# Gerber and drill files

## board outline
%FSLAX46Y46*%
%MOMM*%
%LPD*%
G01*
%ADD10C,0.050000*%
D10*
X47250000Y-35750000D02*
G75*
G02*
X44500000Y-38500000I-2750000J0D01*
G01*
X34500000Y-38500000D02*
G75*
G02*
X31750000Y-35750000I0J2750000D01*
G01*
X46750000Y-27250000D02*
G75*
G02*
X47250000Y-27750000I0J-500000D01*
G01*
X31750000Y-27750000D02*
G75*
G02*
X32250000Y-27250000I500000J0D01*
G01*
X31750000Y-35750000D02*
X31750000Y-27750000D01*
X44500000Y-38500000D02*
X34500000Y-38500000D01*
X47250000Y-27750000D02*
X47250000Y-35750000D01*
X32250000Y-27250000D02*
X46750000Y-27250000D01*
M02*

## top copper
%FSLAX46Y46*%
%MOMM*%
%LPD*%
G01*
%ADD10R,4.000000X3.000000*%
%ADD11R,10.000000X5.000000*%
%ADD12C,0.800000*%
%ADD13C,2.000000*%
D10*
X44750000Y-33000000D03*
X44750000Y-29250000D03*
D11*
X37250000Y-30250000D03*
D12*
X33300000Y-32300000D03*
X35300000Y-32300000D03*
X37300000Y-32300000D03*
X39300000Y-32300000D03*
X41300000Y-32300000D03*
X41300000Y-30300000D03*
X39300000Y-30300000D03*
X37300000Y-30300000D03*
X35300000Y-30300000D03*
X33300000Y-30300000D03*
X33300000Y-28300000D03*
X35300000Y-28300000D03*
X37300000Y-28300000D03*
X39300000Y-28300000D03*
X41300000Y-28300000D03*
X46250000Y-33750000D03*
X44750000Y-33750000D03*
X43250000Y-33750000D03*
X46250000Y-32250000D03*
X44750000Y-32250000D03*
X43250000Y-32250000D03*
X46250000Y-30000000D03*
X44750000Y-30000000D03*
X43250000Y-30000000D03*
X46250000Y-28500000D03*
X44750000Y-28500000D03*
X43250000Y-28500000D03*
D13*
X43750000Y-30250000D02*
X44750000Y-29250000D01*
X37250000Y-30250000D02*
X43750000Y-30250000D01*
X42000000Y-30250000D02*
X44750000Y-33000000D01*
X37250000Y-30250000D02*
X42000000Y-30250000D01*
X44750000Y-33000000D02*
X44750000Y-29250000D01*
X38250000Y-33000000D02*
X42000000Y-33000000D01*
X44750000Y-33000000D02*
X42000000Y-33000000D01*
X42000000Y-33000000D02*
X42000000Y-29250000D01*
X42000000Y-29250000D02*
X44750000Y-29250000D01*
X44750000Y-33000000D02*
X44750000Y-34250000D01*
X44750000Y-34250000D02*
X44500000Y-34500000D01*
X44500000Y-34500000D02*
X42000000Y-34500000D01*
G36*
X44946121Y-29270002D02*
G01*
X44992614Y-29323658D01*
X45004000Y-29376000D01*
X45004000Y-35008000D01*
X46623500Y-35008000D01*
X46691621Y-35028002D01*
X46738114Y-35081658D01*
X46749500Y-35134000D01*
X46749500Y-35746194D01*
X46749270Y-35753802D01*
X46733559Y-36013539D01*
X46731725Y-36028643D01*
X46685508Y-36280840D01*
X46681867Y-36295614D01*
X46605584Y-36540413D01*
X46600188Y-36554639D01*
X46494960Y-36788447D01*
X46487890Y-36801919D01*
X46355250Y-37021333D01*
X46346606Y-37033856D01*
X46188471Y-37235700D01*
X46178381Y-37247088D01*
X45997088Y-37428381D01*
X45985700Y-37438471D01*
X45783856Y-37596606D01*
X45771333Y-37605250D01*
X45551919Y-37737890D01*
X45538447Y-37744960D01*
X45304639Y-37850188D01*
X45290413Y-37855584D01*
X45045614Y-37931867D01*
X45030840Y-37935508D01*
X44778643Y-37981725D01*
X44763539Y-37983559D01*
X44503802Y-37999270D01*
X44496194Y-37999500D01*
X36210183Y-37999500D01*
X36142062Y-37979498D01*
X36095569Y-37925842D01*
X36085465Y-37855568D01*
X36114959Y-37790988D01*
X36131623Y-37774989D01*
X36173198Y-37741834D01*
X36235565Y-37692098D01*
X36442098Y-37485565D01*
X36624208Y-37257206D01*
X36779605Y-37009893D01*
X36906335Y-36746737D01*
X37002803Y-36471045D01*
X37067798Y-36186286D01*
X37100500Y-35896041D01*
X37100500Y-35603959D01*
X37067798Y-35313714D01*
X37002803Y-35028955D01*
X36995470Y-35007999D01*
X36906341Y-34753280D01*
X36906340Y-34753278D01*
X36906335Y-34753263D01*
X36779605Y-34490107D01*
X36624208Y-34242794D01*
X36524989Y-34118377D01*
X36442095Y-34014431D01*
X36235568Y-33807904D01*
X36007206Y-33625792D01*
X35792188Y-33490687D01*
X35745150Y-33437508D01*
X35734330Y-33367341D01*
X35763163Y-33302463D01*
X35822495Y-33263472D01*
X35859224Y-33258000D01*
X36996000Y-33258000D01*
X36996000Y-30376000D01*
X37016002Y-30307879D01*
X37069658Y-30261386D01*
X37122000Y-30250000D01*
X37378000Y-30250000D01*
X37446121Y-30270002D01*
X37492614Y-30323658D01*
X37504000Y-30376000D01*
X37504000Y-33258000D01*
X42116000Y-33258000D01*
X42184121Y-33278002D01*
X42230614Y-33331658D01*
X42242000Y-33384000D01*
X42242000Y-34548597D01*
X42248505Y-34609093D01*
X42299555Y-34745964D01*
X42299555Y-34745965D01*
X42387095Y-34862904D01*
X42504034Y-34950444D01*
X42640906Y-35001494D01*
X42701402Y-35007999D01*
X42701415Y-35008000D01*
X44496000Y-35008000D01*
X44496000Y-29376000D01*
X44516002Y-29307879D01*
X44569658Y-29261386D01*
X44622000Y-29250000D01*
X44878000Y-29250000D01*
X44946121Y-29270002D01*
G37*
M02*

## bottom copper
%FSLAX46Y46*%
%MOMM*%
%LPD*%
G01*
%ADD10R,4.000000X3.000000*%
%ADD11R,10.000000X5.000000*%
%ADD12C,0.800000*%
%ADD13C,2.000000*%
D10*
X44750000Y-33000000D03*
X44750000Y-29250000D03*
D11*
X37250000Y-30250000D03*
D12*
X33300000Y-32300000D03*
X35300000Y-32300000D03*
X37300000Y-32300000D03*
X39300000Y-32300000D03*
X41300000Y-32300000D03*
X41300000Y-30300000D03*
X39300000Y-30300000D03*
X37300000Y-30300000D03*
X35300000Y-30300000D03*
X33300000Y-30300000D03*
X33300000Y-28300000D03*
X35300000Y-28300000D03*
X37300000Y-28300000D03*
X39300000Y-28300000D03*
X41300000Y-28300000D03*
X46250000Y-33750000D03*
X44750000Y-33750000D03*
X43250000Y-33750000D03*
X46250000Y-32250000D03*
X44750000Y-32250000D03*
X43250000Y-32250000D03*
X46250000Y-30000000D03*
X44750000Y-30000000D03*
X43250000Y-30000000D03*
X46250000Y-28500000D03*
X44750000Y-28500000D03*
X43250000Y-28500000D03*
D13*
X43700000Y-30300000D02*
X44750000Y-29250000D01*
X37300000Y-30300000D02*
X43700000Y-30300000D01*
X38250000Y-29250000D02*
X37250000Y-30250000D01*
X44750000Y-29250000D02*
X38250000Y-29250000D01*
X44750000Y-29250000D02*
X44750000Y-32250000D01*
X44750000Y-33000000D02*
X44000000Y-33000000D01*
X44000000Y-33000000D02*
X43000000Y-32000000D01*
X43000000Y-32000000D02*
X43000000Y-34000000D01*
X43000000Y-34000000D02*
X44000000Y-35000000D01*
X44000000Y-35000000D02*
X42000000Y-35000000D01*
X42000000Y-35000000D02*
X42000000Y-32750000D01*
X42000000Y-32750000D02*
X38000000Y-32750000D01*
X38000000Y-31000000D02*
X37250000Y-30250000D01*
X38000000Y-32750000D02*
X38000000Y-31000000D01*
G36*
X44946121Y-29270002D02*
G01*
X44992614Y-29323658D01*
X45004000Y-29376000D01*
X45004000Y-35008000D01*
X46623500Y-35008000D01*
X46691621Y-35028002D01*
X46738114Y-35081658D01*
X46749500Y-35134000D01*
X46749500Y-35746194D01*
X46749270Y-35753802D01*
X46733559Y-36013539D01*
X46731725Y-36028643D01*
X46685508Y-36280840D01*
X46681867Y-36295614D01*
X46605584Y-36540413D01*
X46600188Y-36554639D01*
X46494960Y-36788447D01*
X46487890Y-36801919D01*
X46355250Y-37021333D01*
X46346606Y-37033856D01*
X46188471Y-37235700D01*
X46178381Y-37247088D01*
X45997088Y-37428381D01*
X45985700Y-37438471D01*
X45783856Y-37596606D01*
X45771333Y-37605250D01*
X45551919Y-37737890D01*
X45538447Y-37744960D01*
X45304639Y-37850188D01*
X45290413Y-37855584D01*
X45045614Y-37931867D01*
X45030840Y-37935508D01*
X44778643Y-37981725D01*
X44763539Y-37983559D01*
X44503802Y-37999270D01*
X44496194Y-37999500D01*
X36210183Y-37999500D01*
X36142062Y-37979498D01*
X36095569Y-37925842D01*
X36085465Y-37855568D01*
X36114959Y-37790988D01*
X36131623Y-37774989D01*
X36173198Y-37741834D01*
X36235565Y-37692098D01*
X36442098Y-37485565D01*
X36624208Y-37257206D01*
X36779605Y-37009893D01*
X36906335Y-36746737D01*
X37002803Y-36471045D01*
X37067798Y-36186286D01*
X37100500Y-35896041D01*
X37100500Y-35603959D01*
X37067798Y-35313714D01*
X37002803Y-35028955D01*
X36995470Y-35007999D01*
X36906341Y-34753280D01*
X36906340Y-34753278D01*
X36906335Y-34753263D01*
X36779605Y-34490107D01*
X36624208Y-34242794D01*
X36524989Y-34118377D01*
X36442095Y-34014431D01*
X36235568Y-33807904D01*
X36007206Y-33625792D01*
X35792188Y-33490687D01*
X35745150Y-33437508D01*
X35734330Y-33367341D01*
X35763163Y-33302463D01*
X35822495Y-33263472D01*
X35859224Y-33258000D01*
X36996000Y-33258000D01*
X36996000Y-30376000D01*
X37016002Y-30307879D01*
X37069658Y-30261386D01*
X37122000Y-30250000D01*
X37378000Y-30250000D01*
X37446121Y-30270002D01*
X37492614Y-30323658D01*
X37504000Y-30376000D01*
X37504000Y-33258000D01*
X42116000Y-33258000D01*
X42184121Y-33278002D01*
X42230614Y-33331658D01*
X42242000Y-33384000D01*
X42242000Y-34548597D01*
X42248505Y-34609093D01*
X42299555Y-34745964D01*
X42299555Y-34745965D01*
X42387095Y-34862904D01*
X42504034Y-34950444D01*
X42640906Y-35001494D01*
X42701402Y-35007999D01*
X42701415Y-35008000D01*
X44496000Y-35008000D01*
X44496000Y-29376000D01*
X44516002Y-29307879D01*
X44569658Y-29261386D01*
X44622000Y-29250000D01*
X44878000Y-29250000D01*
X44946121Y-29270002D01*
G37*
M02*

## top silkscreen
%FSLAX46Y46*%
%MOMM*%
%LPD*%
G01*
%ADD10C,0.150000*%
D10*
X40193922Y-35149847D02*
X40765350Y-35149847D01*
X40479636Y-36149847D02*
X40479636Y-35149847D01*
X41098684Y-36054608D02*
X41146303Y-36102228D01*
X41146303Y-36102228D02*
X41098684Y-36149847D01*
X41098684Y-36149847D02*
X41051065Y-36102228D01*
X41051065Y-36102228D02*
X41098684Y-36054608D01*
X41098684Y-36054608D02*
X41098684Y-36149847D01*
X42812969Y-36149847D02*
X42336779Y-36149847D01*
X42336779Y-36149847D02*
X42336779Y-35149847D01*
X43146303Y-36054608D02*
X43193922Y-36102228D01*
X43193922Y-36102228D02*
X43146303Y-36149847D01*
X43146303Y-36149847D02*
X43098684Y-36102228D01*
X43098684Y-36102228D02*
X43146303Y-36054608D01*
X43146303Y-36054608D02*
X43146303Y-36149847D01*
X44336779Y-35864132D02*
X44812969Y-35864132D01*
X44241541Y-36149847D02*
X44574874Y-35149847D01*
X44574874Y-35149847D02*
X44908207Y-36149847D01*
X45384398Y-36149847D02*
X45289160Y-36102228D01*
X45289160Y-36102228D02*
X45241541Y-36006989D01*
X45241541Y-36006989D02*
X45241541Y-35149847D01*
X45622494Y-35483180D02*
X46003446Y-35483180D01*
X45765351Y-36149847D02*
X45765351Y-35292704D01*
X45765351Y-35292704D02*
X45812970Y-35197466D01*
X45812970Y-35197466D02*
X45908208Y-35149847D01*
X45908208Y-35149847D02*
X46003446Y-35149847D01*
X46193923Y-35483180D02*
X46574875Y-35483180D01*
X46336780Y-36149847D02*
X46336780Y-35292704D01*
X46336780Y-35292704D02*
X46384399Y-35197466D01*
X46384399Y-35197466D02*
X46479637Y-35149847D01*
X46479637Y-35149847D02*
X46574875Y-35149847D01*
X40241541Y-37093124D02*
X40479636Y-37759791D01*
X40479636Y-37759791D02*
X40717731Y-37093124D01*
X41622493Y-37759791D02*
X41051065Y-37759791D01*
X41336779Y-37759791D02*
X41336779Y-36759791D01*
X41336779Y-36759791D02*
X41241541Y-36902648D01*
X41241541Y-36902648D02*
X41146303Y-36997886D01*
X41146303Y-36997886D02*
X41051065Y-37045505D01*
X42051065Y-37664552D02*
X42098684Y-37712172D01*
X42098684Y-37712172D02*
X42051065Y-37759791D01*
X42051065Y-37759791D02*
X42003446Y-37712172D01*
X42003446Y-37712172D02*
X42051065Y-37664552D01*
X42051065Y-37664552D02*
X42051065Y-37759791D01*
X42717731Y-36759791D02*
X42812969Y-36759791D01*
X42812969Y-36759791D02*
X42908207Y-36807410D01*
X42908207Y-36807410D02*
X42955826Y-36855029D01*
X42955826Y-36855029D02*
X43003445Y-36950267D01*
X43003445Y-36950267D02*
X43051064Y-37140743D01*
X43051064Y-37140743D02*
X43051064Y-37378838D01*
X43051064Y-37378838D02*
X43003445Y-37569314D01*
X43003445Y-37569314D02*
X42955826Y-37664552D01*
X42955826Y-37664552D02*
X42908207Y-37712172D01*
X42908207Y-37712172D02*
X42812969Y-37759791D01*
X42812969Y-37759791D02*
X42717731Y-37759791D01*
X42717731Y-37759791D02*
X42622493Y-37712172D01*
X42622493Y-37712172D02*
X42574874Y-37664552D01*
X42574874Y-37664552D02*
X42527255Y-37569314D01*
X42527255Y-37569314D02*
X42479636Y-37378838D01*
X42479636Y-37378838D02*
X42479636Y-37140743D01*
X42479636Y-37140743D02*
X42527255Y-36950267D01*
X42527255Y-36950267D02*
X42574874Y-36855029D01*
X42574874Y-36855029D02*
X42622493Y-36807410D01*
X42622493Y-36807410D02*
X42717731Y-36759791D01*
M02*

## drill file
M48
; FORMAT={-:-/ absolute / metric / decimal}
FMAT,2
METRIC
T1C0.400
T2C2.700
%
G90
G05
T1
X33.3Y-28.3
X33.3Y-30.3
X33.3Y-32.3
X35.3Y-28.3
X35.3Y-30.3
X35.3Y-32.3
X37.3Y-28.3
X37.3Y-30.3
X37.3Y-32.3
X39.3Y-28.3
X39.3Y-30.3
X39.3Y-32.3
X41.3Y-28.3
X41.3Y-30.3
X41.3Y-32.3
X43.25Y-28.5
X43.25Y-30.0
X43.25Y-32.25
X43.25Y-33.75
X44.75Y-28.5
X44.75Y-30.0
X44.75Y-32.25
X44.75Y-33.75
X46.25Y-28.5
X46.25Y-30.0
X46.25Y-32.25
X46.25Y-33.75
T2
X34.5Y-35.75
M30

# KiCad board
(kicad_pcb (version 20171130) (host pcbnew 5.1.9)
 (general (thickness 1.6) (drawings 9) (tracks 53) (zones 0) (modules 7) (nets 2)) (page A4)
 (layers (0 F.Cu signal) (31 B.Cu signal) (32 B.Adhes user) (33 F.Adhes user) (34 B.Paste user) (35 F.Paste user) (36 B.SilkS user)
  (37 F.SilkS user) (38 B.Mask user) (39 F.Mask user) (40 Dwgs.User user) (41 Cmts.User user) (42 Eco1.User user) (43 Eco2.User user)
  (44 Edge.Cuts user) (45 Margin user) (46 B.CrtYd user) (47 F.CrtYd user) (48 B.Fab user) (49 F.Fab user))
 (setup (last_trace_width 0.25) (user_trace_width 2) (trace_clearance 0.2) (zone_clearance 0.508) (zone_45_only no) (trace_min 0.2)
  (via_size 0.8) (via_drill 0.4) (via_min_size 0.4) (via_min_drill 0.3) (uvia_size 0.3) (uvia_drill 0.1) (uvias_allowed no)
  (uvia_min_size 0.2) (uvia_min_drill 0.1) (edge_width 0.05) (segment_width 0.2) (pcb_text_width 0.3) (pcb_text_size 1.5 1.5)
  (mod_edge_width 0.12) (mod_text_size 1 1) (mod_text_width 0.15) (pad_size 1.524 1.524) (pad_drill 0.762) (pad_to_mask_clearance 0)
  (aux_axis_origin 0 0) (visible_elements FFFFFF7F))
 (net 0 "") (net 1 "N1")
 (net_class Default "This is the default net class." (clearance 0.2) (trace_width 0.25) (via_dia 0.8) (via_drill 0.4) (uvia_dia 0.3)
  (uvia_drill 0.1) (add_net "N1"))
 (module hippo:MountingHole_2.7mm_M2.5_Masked (layer F.Cu) (at 34.5 35.75)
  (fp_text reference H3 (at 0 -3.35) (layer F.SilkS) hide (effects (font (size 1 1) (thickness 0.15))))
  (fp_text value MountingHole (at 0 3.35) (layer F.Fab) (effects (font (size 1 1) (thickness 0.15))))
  (pad "" np_thru_hole circle (at 0 0) (size 2.7 2.7) (drill 2.7) (layers *.Cu *.Mask) (solder_mask_margin 1) (clearance 1.25)))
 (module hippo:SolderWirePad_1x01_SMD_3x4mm (layer B.Cu) (at 44.75 33 90)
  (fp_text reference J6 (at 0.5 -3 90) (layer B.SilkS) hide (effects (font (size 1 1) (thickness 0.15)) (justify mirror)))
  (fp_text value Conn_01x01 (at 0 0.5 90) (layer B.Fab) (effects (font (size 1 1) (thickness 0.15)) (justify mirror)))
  (pad 1 smd rect (at 0 0 90) (size 3 4) (layers B.Cu B.Paste B.Mask) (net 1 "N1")))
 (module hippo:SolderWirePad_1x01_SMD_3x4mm (layer B.Cu) (at 44.75 29.25 90)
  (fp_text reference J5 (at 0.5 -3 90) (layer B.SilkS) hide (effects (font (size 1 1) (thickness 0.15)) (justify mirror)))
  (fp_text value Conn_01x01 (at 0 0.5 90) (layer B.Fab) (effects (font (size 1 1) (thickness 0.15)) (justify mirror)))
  (pad 1 smd rect (at 0 0 90) (size 3 4) (layers B.Cu B.Paste B.Mask) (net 1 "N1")))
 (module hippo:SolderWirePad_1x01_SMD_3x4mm (layer F.Cu) (at 44.75 33 90)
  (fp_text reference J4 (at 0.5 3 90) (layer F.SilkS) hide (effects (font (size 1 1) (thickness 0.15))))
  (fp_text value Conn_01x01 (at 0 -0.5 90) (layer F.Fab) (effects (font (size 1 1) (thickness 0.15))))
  (pad 1 smd rect (at 0 0 90) (size 3 4) (layers F.Cu F.Paste F.Mask) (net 1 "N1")))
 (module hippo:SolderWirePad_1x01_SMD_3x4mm (layer F.Cu) (at 44.75 29.25 90)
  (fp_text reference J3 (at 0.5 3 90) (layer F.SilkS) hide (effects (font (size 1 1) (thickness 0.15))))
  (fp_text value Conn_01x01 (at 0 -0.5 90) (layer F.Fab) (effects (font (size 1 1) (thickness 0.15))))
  (pad 1 smd rect (at 0 0 90) (size 3 4) (layers F.Cu F.Paste F.Mask) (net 1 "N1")))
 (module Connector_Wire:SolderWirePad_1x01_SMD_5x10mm (layer B.Cu) (at 37.25 30.25 90)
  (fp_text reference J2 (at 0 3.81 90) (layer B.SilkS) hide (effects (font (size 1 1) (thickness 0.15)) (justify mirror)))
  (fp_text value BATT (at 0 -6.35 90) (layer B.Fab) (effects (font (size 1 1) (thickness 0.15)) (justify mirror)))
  (pad 1 smd rect (at 0 0 90) (size 5 10) (layers B.Cu B.Paste B.Mask) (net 1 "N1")))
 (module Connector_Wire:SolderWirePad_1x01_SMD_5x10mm (layer F.Cu) (at 37.25 30.25 90)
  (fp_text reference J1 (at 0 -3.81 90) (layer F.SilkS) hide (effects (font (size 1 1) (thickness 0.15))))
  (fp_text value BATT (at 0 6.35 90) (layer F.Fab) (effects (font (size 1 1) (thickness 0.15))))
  (pad 1 smd rect (at 0 0 90) (size 5 10) (layers F.Cu F.Paste F.Mask) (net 1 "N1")))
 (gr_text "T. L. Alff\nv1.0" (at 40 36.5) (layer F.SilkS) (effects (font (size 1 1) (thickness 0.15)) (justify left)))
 (gr_arc (start 44.5 35.75) (end 44.5 38.5) (angle -90) (layer Edge.Cuts) (width 0.05))
 (gr_arc (start 34.5 35.75) (end 31.75 35.75) (angle -90) (layer Edge.Cuts) (width 0.05))
 (gr_arc (start 46.75 27.75) (end 47.25 27.75) (angle -90) (layer Edge.Cuts) (width 0.05))
 (gr_arc (start 32.25 27.75) (end 32.25 27.25) (angle -90) (layer Edge.Cuts) (width 0.05))
 (gr_line (start 31.75 35.75) (end 31.75 27.75) (layer Edge.Cuts) (width 0.05))
 (gr_line (start 44.5 38.5) (end 34.5 38.5) (layer Edge.Cuts) (width 0.05))
 (gr_line (start 47.25 27.75) (end 47.25 35.75) (layer Edge.Cuts) (width 0.05))
 (gr_line (start 32.25 27.25) (end 46.75 27.25) (layer Edge.Cuts) (width 0.05))
 (via (at 33.3 32.3) (size 0.8) (drill 0.4) (layers F.Cu B.Cu) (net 1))
 (via (at 35.3 32.3) (size 0.8) (drill 0.4) (layers F.Cu B.Cu) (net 1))
 (via (at 37.3 32.3) (size 0.8) (drill 0.4) (layers F.Cu B.Cu) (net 1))
 (via (at 39.3 32.3) (size 0.8) (drill 0.4) (layers F.Cu B.Cu) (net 1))
 (via (at 41.3 32.3) (size 0.8) (drill 0.4) (layers F.Cu B.Cu) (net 1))
 (via (at 41.3 30.3) (size 0.8) (drill 0.4) (layers F.Cu B.Cu) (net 1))
 (via (at 39.3 30.3) (size 0.8) (drill 0.4) (layers F.Cu B.Cu) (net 1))
 (via (at 37.3 30.3) (size 0.8) (drill 0.4) (layers F.Cu B.Cu) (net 1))
 (via (at 35.3 30.3) (size 0.8) (drill 0.4) (layers F.Cu B.Cu) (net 1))
 (via (at 33.3 30.3) (size 0.8) (drill 0.4) (layers F.Cu B.Cu) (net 1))
 (via (at 33.3 28.3) (size 0.8) (drill 0.4) (layers F.Cu B.Cu) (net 1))
 (via (at 35.3 28.3) (size 0.8) (drill 0.4) (layers F.Cu B.Cu) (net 1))
 (via (at 37.3 28.3) (size 0.8) (drill 0.4) (layers F.Cu B.Cu) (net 1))
 (via (at 39.3 28.3) (size 0.8) (drill 0.4) (layers F.Cu B.Cu) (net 1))
 (via (at 41.3 28.3) (size 0.8) (drill 0.4) (layers F.Cu B.Cu) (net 1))
 (via (at 46.25 33.75) (size 0.8) (drill 0.4) (layers F.Cu B.Cu) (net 1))
 (via (at 44.75 33.75) (size 0.8) (drill 0.4) (layers F.Cu B.Cu) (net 1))
 (via (at 43.25 33.75) (size 0.8) (drill 0.4) (layers F.Cu B.Cu) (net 1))
 (via (at 46.25 32.25) (size 0.8) (drill 0.4) (layers F.Cu B.Cu) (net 1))
 (via (at 44.75 32.25) (size 0.8) (drill 0.4) (layers F.Cu B.Cu) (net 1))
 (via (at 43.25 32.25) (size 0.8) (drill 0.4) (layers F.Cu B.Cu) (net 1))
 (via (at 46.25 30) (size 0.8) (drill 0.4) (layers F.Cu B.Cu) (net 1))
 (via (at 44.75 30) (size 0.8) (drill 0.4) (layers F.Cu B.Cu) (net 1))
 (via (at 43.25 30) (size 0.8) (drill 0.4) (layers F.Cu B.Cu) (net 1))
 (via (at 46.25 28.5) (size 0.8) (drill 0.4) (layers F.Cu B.Cu) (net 1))
 (via (at 44.75 28.5) (size 0.8) (drill 0.4) (layers F.Cu B.Cu) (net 1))
 (via (at 43.25 28.5) (size 0.8) (drill 0.4) (layers F.Cu B.Cu) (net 1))
 (segment (start 43.75 30.25) (end 44.75 29.25) (width 2) (layer F.Cu) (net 1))
 (segment (start 37.25 30.25) (end 43.75 30.25) (width 2) (layer F.Cu) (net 1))
 (segment (start 42 30.25) (end 44.75 33) (width 2) (layer F.Cu) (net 1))
 (segment (start 37.25 30.25) (end 42 30.25) (width 2) (layer F.Cu) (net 1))
 (segment (start 44.75 33) (end 44.75 29.25) (width 2) (layer F.Cu) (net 1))
 (segment (start 38.25 33) (end 42 33) (width 2) (layer F.Cu) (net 1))
 (segment (start 44.75 33) (end 42 33) (width 2) (layer F.Cu) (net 1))
 (segment (start 42 33) (end 42 29.25) (width 2) (layer F.Cu) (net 1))
 (segment (start 42 29.25) (end 44.75 29.25) (width 2) (layer F.Cu) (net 1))
 (segment (start 44.75 33) (end 44.75 34.25) (width 2) (layer F.Cu) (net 1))
 (segment (start 44.75 34.25) (end 44.5 34.5) (width 2) (layer F.Cu) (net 1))
 (segment (start 44.5 34.5) (end 42 34.5) (width 2) (layer F.Cu) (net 1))
 (segment (start 43.7 30.3) (end 44.75 29.25) (width 2) (layer B.Cu) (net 1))
 (segment (start 37.3 30.3) (end 43.7 30.3) (width 2) (layer B.Cu) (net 1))
 (segment (start 38.25 29.25) (end 37.25 30.25) (width 2) (layer B.Cu) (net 1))
 (segment (start 44.75 29.25) (end 38.25 29.25) (width 2) (layer B.Cu) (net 1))
 (segment (start 44.75 29.25) (end 44.75 32.25) (width 2) (layer B.Cu) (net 1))
 (segment (start 44.75 33) (end 44 33) (width 2) (layer B.Cu) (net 1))
 (segment (start 44 33) (end 43 32) (width 2) (layer B.Cu) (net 1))
 (segment (start 43 32) (end 43 34) (width 2) (layer B.Cu) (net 1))
 (segment (start 43 34) (end 44 35) (width 2) (layer B.Cu) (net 1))
 (segment (start 44 35) (end 42 35) (width 2) (layer B.Cu) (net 1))
 (segment (start 42 35) (end 42 32.75) (width 2) (layer B.Cu) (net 1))
 (segment (start 42 32.75) (end 38 32.75) (width 2) (layer B.Cu) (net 1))
 (segment (start 38 31) (end 37.25 30.25) (width 2) (layer B.Cu) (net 1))
 (segment (start 38 32.75) (end 38 31) (width 2) (layer B.Cu) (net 1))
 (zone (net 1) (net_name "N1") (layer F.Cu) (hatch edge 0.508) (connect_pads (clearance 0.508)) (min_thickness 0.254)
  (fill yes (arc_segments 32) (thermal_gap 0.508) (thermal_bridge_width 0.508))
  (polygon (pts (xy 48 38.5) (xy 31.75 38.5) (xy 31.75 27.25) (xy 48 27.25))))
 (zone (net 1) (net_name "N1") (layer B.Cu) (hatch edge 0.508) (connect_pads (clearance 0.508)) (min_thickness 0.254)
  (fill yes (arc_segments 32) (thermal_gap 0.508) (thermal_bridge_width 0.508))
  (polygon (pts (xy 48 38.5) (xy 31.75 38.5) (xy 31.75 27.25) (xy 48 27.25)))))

